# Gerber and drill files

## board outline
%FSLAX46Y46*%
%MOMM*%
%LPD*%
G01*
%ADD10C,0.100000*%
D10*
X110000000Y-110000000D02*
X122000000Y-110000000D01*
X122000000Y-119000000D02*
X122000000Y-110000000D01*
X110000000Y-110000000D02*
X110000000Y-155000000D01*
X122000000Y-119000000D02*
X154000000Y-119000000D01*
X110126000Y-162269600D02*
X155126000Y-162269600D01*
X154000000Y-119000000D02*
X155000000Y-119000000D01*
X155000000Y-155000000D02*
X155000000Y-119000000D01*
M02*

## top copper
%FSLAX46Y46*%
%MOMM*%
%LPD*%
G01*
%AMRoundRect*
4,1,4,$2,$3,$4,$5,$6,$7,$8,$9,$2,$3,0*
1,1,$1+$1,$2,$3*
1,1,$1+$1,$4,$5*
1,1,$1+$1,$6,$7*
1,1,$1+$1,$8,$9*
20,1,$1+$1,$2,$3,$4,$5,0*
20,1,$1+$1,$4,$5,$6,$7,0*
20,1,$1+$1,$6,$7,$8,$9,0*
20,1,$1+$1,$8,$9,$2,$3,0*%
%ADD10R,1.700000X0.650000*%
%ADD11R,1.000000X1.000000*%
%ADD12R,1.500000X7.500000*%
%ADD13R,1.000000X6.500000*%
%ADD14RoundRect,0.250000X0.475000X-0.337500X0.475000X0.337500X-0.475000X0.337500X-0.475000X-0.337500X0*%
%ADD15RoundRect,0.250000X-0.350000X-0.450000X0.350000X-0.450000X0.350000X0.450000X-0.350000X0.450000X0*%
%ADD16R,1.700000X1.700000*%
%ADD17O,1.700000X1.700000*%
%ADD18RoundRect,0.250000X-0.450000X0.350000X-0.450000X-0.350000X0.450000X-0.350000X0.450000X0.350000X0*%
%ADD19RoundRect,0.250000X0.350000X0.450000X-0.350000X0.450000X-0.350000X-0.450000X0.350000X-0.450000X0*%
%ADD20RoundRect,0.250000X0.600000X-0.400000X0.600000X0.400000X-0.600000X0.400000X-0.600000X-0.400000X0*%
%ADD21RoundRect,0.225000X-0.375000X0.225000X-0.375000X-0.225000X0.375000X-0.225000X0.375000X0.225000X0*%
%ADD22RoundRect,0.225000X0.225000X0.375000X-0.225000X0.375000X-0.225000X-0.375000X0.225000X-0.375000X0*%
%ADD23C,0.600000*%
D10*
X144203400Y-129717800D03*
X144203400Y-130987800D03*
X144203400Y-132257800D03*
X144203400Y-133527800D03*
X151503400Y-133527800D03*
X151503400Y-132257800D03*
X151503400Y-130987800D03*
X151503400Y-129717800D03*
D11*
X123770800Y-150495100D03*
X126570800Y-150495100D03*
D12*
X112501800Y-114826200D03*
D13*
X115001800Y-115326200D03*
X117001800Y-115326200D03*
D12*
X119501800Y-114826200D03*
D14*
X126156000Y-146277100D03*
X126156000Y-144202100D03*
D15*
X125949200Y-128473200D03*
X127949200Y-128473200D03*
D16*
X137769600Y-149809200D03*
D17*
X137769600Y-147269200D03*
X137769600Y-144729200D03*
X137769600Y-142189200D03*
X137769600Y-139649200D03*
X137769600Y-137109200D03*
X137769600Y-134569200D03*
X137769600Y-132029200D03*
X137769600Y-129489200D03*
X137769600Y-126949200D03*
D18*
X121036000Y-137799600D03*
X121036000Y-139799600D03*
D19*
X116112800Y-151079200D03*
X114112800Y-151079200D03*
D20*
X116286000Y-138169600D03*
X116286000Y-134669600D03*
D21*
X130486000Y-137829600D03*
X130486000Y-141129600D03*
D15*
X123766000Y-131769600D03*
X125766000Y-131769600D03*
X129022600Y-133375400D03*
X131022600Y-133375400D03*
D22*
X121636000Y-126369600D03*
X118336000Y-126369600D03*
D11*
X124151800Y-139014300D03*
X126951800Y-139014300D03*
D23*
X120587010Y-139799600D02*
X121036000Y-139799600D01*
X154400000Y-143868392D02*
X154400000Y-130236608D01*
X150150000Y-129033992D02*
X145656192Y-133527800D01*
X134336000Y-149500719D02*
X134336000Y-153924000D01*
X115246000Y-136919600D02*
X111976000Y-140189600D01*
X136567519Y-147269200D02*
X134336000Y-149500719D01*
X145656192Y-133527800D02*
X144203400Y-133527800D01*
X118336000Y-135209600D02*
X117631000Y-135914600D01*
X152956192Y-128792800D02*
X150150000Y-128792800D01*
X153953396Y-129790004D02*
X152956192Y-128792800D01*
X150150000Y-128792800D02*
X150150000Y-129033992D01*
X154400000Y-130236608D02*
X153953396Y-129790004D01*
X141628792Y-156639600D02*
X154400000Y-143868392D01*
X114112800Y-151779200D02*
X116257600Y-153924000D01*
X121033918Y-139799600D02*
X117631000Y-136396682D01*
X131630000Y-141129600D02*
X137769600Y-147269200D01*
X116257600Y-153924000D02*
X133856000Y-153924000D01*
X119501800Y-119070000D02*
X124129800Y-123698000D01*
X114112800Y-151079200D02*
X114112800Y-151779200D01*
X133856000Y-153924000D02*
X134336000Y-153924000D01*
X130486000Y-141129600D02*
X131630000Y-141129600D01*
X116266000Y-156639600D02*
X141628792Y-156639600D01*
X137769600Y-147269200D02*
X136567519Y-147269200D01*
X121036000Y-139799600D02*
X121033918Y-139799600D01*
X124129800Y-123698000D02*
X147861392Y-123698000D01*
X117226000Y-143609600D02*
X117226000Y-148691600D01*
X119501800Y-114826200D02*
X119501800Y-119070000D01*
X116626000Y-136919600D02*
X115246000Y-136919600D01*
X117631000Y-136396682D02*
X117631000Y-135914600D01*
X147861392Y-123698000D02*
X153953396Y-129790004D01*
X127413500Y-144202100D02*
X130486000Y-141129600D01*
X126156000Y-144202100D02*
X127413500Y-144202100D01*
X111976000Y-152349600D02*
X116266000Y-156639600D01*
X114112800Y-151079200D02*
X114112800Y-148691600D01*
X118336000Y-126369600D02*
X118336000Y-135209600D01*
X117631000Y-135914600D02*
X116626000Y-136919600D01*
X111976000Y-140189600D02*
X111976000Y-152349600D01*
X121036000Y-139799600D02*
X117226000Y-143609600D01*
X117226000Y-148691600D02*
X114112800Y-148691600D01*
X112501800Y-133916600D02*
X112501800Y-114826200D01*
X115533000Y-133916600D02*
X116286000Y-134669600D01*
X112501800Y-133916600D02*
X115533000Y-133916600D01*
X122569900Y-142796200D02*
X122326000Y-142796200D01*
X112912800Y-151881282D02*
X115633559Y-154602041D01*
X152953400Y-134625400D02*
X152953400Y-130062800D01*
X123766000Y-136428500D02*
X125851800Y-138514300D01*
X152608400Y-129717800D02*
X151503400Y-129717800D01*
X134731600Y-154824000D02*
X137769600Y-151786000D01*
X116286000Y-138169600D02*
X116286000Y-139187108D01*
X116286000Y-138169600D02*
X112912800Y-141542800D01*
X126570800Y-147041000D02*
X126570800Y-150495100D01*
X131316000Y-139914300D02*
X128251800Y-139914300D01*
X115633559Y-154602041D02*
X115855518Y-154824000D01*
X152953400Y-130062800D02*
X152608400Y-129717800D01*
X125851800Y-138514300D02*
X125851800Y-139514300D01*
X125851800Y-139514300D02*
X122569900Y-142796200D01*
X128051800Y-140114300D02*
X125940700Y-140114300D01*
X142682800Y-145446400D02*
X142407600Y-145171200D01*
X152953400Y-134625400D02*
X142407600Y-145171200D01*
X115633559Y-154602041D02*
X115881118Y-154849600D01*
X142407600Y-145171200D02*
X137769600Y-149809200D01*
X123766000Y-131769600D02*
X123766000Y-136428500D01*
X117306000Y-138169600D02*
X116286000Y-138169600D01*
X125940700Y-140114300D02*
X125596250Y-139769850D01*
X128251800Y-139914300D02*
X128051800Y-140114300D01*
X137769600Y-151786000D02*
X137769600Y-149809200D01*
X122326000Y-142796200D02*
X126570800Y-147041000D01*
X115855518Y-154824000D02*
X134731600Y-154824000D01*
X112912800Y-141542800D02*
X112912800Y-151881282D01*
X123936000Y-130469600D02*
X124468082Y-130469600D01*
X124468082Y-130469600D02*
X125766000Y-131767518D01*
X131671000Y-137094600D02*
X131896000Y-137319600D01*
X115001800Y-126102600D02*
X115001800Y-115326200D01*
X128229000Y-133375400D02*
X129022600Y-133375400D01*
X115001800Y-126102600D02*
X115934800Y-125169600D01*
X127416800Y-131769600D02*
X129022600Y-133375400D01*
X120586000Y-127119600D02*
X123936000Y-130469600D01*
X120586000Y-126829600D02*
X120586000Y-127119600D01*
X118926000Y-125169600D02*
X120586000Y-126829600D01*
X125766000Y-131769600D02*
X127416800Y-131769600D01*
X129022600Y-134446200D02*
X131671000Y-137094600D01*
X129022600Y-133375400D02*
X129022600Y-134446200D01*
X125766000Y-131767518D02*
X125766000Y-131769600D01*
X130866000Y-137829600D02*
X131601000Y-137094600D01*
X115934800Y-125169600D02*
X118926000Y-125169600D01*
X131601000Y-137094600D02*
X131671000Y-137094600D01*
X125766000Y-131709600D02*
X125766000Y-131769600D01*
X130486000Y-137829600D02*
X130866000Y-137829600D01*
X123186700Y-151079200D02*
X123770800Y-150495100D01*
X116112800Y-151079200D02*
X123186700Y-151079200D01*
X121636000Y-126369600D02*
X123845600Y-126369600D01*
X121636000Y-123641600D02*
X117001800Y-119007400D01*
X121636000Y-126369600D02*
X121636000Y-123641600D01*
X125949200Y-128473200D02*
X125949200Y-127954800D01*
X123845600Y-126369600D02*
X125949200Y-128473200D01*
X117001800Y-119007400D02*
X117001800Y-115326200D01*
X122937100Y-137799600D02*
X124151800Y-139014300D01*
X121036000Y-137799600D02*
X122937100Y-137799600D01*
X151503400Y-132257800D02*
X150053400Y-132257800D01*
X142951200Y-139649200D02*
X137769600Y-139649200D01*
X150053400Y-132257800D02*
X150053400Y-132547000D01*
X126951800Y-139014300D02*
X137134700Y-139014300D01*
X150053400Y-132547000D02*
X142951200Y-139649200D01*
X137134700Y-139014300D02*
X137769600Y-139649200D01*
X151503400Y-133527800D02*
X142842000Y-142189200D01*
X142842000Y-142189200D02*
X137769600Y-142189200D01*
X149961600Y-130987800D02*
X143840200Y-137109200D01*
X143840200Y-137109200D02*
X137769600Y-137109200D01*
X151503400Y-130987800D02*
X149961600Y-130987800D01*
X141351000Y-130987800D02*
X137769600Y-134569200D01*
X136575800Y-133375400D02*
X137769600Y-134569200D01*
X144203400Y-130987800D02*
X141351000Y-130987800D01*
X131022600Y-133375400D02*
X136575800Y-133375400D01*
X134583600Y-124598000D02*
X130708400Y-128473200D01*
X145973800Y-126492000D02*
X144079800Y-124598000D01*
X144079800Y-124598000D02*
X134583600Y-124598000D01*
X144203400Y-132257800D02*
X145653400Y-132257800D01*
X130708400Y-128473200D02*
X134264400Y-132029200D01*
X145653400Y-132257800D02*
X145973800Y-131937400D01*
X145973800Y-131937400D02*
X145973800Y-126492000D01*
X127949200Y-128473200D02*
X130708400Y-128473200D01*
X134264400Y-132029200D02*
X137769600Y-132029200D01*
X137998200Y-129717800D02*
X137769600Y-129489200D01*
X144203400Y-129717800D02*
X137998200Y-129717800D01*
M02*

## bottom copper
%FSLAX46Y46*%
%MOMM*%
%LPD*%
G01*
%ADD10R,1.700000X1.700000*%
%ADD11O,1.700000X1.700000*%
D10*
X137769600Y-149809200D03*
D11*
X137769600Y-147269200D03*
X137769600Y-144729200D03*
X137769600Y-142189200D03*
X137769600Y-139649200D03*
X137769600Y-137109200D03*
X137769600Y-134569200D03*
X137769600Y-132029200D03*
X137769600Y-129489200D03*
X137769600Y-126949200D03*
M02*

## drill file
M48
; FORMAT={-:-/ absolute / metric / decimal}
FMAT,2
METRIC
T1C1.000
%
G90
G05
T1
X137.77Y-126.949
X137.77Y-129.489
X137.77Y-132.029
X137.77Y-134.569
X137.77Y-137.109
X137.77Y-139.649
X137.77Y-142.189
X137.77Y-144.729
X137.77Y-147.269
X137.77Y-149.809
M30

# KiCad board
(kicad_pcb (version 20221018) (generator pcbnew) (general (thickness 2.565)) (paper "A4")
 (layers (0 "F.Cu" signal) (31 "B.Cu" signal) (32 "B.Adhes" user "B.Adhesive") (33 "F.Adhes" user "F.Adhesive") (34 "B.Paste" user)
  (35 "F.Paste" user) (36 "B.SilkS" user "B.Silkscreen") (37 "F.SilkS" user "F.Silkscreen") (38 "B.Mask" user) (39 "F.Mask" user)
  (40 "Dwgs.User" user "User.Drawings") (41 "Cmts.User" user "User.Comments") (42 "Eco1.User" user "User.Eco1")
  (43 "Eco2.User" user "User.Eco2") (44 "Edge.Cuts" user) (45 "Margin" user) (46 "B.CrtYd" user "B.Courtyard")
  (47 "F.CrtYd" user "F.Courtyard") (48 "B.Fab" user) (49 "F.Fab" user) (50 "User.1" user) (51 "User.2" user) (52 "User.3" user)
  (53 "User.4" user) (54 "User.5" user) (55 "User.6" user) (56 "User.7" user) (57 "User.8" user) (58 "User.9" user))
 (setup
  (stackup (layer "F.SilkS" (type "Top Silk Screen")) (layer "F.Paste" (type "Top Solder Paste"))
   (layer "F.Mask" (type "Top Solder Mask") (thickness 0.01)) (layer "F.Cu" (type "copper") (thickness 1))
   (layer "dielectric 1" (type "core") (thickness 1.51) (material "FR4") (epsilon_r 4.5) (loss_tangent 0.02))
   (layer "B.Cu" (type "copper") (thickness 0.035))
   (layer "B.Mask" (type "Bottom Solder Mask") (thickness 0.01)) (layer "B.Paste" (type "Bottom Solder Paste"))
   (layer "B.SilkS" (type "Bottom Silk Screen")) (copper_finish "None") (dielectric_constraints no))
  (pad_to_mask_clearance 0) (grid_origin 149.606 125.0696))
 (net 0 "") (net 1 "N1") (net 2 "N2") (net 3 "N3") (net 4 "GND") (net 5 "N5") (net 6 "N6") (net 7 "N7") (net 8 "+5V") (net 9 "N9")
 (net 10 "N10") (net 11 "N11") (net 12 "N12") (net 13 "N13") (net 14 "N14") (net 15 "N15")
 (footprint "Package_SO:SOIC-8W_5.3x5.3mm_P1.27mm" (layer "F.Cu") (at 147.8534 131.6228)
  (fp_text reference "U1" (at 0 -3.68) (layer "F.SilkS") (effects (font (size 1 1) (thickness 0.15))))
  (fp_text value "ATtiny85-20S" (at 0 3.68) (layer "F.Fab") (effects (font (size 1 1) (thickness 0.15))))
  (pad "1" smd rect (at -3.65 -1.905) (size 1.7 0.65) (layers "F.Cu" "F.Paste" "F.Mask") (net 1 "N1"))
  (pad "2" smd rect (at -3.65 -0.635) (size 1.7 0.65) (layers "F.Cu" "F.Paste" "F.Mask") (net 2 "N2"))
  (pad "3" smd rect (at -3.65 0.635) (size 1.7 0.65) (layers "F.Cu" "F.Paste" "F.Mask") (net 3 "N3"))
  (pad "4" smd rect (at -3.65 1.905) (size 1.7 0.65) (layers "F.Cu" "F.Paste" "F.Mask") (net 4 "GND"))
  (pad "5" smd rect (at 3.65 1.905) (size 1.7 0.65) (layers "F.Cu" "F.Paste" "F.Mask") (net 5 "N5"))
  (pad "6" smd rect (at 3.65 0.635) (size 1.7 0.65) (layers "F.Cu" "F.Paste" "F.Mask") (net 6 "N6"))
  (pad "7" smd rect (at 3.65 -0.635) (size 1.7 0.65) (layers "F.Cu" "F.Paste" "F.Mask") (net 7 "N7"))
  (pad "8" smd rect (at 3.65 -1.905) (size 1.7 0.65) (layers "F.Cu" "F.Paste" "F.Mask") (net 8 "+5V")))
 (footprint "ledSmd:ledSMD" (layer "F.Cu") (at 125.5708 150.4951)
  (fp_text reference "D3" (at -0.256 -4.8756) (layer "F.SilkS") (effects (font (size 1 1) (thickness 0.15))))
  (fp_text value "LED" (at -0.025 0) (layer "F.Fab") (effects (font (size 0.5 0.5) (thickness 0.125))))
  (pad "1" smd rect (at -1.8 0) (size 1 1) (layers "F.Cu" "F.Paste" "F.Mask") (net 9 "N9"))
  (pad "2" smd rect (at 1 0) (size 1 1) (layers "F.Cu" "F.Paste" "F.Mask") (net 8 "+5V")))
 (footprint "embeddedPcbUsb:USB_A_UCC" (layer "F.Cu") (at 116.0018 115.0262 -90)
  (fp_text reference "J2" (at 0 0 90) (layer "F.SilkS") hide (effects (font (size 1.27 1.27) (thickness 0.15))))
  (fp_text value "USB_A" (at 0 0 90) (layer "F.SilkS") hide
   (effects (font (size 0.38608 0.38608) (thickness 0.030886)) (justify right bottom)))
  (pad "1" smd rect (at -0.2 3.5 270) (size 7.5 1.5) (layers "F.Cu" "F.Paste" "F.Mask") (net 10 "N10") (solder_mask_margin 0.1016))
  (pad "2" smd rect (at 0.3 1 270) (size 6.5 1) (layers "F.Cu" "F.Paste" "F.Mask") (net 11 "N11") (solder_mask_margin 0.1016))
  (pad "3" smd rect (at 0.3 -1 270) (size 6.5 1) (layers "F.Cu" "F.Paste" "F.Mask") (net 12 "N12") (solder_mask_margin 0.1016))
  (pad "4" smd rect (at -0.2 -3.5 270) (size 7.5 1.5) (layers "F.Cu" "F.Paste" "F.Mask") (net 4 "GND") (solder_mask_margin 0.1016)))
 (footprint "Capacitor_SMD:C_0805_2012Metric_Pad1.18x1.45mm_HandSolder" (layer "F.Cu") (at 126.156 145.2396 90)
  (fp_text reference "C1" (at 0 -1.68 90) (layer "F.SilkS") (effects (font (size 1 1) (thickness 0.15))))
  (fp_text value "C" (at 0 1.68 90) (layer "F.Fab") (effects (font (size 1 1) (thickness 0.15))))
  (pad "1" smd roundrect (at -1.0375 0 90) (size 1.175 1.45) (layers "F.Cu" "F.Paste" "F.Mask") (roundrect_rratio 0.212766) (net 8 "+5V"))
  (pad "2" smd roundrect (at 1.0375 0 90) (size 1.175 1.45) (layers "F.Cu" "F.Paste" "F.Mask") (roundrect_rratio 0.212766) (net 4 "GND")))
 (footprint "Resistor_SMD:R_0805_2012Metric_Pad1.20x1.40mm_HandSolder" (layer "F.Cu") (at 126.9492 128.4732)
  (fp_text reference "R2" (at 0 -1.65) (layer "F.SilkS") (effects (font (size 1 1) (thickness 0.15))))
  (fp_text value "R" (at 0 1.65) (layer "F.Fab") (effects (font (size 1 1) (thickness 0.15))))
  (pad "1" smd roundrect (at -1 0) (size 1.2 1.4) (layers "F.Cu" "F.Paste" "F.Mask") (roundrect_rratio 0.208333) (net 12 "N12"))
  (pad "2" smd roundrect (at 1 0) (size 1.2 1.4) (layers "F.Cu" "F.Paste" "F.Mask") (roundrect_rratio 0.208333) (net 3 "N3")))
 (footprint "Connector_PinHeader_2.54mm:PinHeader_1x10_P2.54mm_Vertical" (layer "F.Cu") (at 137.7696 149.8092 180)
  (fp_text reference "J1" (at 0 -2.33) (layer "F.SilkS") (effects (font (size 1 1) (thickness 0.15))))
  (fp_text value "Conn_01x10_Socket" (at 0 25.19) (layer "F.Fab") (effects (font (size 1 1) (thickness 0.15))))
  (pad "1" thru_hole rect (at 0 0 180) (size 1.7 1.7) (drill 1) (layers "*.Cu" "*.Mask") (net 8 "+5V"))
  (pad "2" thru_hole oval (at 0 2.54 180) (size 1.7 1.7) (drill 1) (layers "*.Cu" "*.Mask") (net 4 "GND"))
  (pad "3" thru_hole oval (at 0 5.08 180) (size 1.7 1.7) (drill 1) (layers "*.Cu" "*.Mask") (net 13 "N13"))
  (pad "4" thru_hole oval (at 0 7.62 180) (size 1.7 1.7) (drill 1) (layers "*.Cu" "*.Mask") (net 5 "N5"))
  (pad "5" thru_hole oval (at 0 10.16 180) (size 1.7 1.7) (drill 1) (layers "*.Cu" "*.Mask") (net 6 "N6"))
  (pad "6" thru_hole oval (at 0 12.7 180) (size 1.7 1.7) (drill 1) (layers "*.Cu" "*.Mask") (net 7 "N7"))
  (pad "7" thru_hole oval (at 0 15.24 180) (size 1.7 1.7) (drill 1) (layers "*.Cu" "*.Mask") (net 2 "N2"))
  (pad "8" thru_hole oval (at 0 17.78 180) (size 1.7 1.7) (drill 1) (layers "*.Cu" "*.Mask") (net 3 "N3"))
  (pad "9" thru_hole oval (at 0 20.32 180) (size 1.7 1.7) (drill 1) (layers "*.Cu" "*.Mask") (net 1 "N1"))
  (pad "10" thru_hole oval (at 0 22.86 180) (size 1.7 1.7) (drill 1) (layers "*.Cu" "*.Mask") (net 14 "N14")))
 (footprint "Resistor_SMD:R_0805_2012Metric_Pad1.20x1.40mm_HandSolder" (layer "F.Cu") (at 121.036 138.7996 -90)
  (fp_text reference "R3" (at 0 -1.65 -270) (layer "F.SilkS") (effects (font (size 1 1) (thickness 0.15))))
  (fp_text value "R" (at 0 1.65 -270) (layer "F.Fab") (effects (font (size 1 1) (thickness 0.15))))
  (pad "1" smd roundrect (at -1 0 270) (size 1.2 1.4) (layers "F.Cu" "F.Paste" "F.Mask") (roundrect_rratio 0.208333) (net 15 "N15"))
  (pad "2" smd roundrect (at 1 0 270) (size 1.2 1.4) (layers "F.Cu" "F.Paste" "F.Mask") (roundrect_rratio 0.208333) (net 4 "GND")))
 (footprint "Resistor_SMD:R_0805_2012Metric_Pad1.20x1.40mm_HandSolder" (layer "F.Cu") (at 115.1128 151.0792 180)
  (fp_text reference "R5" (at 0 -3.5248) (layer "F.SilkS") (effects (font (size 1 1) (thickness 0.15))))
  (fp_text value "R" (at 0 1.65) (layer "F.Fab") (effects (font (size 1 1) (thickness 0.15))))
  (pad "1" smd roundrect (at -1 0 180) (size 1.2 1.4) (layers "F.Cu" "F.Paste" "F.Mask") (roundrect_rratio 0.208333) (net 9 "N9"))
  (pad "2" smd roundrect (at 1 0 180) (size 1.2 1.4) (layers "F.Cu" "F.Paste" "F.Mask") (roundrect_rratio 0.208333) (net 4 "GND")))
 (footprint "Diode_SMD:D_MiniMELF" (layer "F.Cu") (at 116.286 136.4196 90)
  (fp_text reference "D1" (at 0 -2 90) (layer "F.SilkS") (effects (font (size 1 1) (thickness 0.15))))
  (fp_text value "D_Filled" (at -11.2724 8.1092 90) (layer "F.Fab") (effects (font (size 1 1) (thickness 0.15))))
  (pad "1" smd roundrect (at -1.75 0 90) (size 1.3 1.7) (layers "F.Cu" "F.Paste" "F.Mask") (roundrect_rratio 0.1923076923) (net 8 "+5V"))
  (pad "2" smd roundrect (at 1.75 0 90) (size 1.3 1.7) (layers "F.Cu" "F.Paste" "F.Mask") (roundrect_rratio 0.1923076923) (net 10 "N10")))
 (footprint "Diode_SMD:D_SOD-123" (layer "F.Cu") (at 130.486 139.4796 -90)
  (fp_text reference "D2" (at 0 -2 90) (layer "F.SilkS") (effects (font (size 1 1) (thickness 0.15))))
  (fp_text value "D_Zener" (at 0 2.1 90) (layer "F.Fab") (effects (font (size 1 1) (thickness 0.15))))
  (pad "1" smd roundrect (at -1.65 0 270) (size 0.9 1.2) (layers "F.Cu" "F.Paste" "F.Mask") (roundrect_rratio 0.25) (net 11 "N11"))
  (pad "2" smd roundrect (at 1.65 0 270) (size 0.9 1.2) (layers "F.Cu" "F.Paste" "F.Mask") (roundrect_rratio 0.25) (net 4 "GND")))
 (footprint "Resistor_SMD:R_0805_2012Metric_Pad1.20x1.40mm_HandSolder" (layer "F.Cu") (at 124.766 131.7696)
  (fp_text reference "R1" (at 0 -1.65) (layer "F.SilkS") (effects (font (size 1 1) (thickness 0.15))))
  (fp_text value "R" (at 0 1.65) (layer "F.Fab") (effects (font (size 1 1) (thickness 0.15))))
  (pad "1" smd roundrect (at -1 0) (size 1.2 1.4) (layers "F.Cu" "F.Paste" "F.Mask") (roundrect_rratio 0.208333) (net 8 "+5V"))
  (pad "2" smd roundrect (at 1 0) (size 1.2 1.4) (layers "F.Cu" "F.Paste" "F.Mask") (roundrect_rratio 0.208333) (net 11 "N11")))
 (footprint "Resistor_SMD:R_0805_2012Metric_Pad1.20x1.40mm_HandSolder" (layer "F.Cu") (at 130.0226 133.3754)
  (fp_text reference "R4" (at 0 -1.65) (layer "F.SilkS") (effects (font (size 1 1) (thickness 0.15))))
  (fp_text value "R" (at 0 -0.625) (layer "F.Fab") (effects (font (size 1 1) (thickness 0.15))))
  (pad "1" smd roundrect (at -1 0) (size 1.2 1.4) (layers "F.Cu" "F.Paste" "F.Mask") (roundrect_rratio 0.208333) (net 11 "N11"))
  (pad "2" smd roundrect (at 1 0) (size 1.2 1.4) (layers "F.Cu" "F.Paste" "F.Mask") (roundrect_rratio 0.208333) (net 2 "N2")))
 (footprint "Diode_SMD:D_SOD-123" (layer "F.Cu") (at 119.986 126.3696 180)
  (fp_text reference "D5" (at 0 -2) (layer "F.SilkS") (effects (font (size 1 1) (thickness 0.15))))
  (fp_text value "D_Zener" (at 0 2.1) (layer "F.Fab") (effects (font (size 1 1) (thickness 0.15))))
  (pad "1" smd roundrect (at -1.65 0 180) (size 0.9 1.2) (layers "F.Cu" "F.Paste" "F.Mask") (roundrect_rratio 0.25) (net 12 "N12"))
  (pad "2" smd roundrect (at 1.65 0 180) (size 0.9 1.2) (layers "F.Cu" "F.Paste" "F.Mask") (roundrect_rratio 0.25) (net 4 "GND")))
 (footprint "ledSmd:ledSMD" (layer "F.Cu") (at 125.9518 139.0143)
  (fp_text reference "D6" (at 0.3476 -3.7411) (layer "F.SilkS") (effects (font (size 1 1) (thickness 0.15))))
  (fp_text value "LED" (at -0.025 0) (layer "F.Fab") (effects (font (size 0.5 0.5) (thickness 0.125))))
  (pad "1" smd rect (at -1.8 0) (size 1 1) (layers "F.Cu" "F.Paste" "F.Mask") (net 15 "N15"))
  (pad "2" smd rect (at 1 0) (size 1 1) (layers "F.Cu" "F.Paste" "F.Mask") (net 6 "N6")))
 (gr_line (start 110 110) (end 122 110) (stroke (width 0.1) (type default)) (layer "Edge.Cuts"))
 (gr_line (start 122 119) (end 122 110) (stroke (width 0.1) (type default)) (layer "Edge.Cuts"))
 (gr_line (start 110 110) (end 110 155) (stroke (width 0.1) (type default)) (layer "Edge.Cuts"))
 (gr_line (start 122 119) (end 154 119) (stroke (width 0.1) (type default)) (layer "Edge.Cuts"))
 (gr_line (start 110.126 162.2696) (end 155.126 162.2696) (stroke (width 0.1) (type default)) (layer "Edge.Cuts"))
 (gr_line (start 154 119) (end 155 119) (stroke (width 0.1) (type default)) (layer "Edge.Cuts"))
 (gr_line (start 155 155) (end 155 119) (stroke (width 0.1) (type default)) (layer "Edge.Cuts"))
 (segment (start 120.58701 139.7996) (end 121.036 139.7996) (width 0.6) (layer "F.Cu") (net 4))
 (segment (start 154.4 143.868392) (end 154.4 130.236608) (width 0.6) (layer "F.Cu") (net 4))
 (segment (start 150.15 129.033992) (end 145.656192 133.5278) (width 0.6) (layer "F.Cu") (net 4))
 (segment (start 134.336 149.500719) (end 134.336 153.924) (width 0.6) (layer "F.Cu") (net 4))
 (segment (start 115.246 136.9196) (end 111.976 140.1896) (width 0.6) (layer "F.Cu") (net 4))
 (segment (start 136.567519 147.2692) (end 134.336 149.500719) (width 0.6) (layer "F.Cu") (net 4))
 (segment (start 145.656192 133.5278) (end 144.2034 133.5278) (width 0.6) (layer "F.Cu") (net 4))
 (segment (start 118.336 135.2096) (end 117.631 135.9146) (width 0.6) (layer "F.Cu") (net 4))
 (segment (start 152.956192 128.7928) (end 150.15 128.7928) (width 0.6) (layer "F.Cu") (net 4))
 (segment (start 153.953396 129.790004) (end 152.956192 128.7928) (width 0.6) (layer "F.Cu") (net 4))
 (segment (start 150.15 128.7928) (end 150.15 129.033992) (width 0.6) (layer "F.Cu") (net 4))
 (segment (start 154.4 130.236608) (end 153.953396 129.790004) (width 0.6) (layer "F.Cu") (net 4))
 (segment (start 141.628792 156.6396) (end 154.4 143.868392) (width 0.6) (layer "F.Cu") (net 4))
 (segment (start 114.1128 151.7792) (end 116.2576 153.924) (width 0.6) (layer "F.Cu") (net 4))
 (segment (start 121.033918 139.7996) (end 117.631 136.396682) (width 0.6) (layer "F.Cu") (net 4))
 (segment (start 131.63 141.1296) (end 137.7696 147.2692) (width 0.6) (layer "F.Cu") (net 4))
 (segment (start 116.2576 153.924) (end 133.856 153.924) (width 0.6) (layer "F.Cu") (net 4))
 (segment (start 119.5018 119.07) (end 124.1298 123.698) (width 0.6) (layer "F.Cu") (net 4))
 (segment (start 114.1128 151.0792) (end 114.1128 151.7792) (width 0.6) (layer "F.Cu") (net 4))
 (segment (start 133.856 153.924) (end 134.336 153.924) (width 0.6) (layer "F.Cu") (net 4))
 (segment (start 130.486 141.1296) (end 131.63 141.1296) (width 0.6) (layer "F.Cu") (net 4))
 (segment (start 116.266 156.6396) (end 141.628792 156.6396) (width 0.6) (layer "F.Cu") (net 4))
 (segment (start 137.7696 147.2692) (end 136.567519 147.2692) (width 0.6) (layer "F.Cu") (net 4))
 (segment (start 121.036 139.7996) (end 121.033918 139.7996) (width 0.6) (layer "F.Cu") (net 4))
 (segment (start 124.1298 123.698) (end 147.861392 123.698) (width 0.6) (layer "F.Cu") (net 4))
 (segment (start 117.226 143.6096) (end 117.226 148.6916) (width 0.6) (layer "F.Cu") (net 4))
 (segment (start 119.5018 114.8262) (end 119.5018 119.07) (width 0.6) (layer "F.Cu") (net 4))
 (segment (start 116.626 136.9196) (end 115.246 136.9196) (width 0.6) (layer "F.Cu") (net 4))
 (segment (start 117.631 136.396682) (end 117.631 135.9146) (width 0.6) (layer "F.Cu") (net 4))
 (segment (start 147.861392 123.698) (end 153.953396 129.790004) (width 0.6) (layer "F.Cu") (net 4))
 (segment (start 127.4135 144.2021) (end 130.486 141.1296) (width 0.6) (layer "F.Cu") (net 4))
 (segment (start 126.156 144.2021) (end 127.4135 144.2021) (width 0.6) (layer "F.Cu") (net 4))
 (segment (start 111.976 152.3496) (end 116.266 156.6396) (width 0.6) (layer "F.Cu") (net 4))
 (segment (start 114.1128 151.0792) (end 114.1128 148.6916) (width 0.6) (layer "F.Cu") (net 4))
 (segment (start 118.336 126.3696) (end 118.336 135.2096) (width 0.6) (layer "F.Cu") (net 4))
 (segment (start 117.631 135.9146) (end 116.626 136.9196) (width 0.6) (layer "F.Cu") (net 4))
 (segment (start 111.976 140.1896) (end 111.976 152.3496) (width 0.6) (layer "F.Cu") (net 4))
 (segment (start 121.036 139.7996) (end 117.226 143.6096) (width 0.6) (layer "F.Cu") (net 4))
 (segment (start 117.226 148.6916) (end 114.1128 148.6916) (width 0.6) (layer "F.Cu") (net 4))
 (segment (start 112.5018 133.9166) (end 112.5018 114.8262) (width 0.6) (layer "F.Cu") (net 10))
 (segment (start 115.533 133.9166) (end 116.286 134.6696) (width 0.6) (layer "F.Cu") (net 10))
 (segment (start 112.5018 133.9166) (end 115.533 133.9166) (width 0.6) (layer "F.Cu") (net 10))
 (segment (start 122.5699 142.7962) (end 122.326 142.7962) (width 0.6) (layer "F.Cu") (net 8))
 (segment (start 112.9128 151.881282) (end 115.633559 154.602041) (width 0.6) (layer "F.Cu") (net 8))
 (segment (start 152.9534 134.6254) (end 152.9534 130.0628) (width 0.6) (layer "F.Cu") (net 8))
 (segment (start 123.766 136.4285) (end 125.8518 138.5143) (width 0.6) (layer "F.Cu") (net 8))
 (segment (start 152.6084 129.7178) (end 151.5034 129.7178) (width 0.6) (layer "F.Cu") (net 8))
 (segment (start 134.7316 154.824) (end 137.7696 151.786) (width 0.6) (layer "F.Cu") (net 8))
 (segment (start 116.286 138.1696) (end 116.286 139.187108) (width 0.6) (layer "F.Cu") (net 8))
 (segment (start 116.286 138.1696) (end 112.9128 141.5428) (width 0.6) (layer "F.Cu") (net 8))
 (segment (start 126.5708 147.041) (end 126.5708 150.4951) (width 0.6) (layer "F.Cu") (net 8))
 (segment (start 131.316 139.9143) (end 128.2518 139.9143) (width 0.6) (layer "F.Cu") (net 8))
 (segment (start 115.633559 154.602041) (end 115.855518 154.824) (width 0.6) (layer "F.Cu") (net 8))
 (segment (start 152.9534 130.0628) (end 152.6084 129.7178) (width 0.6) (layer "F.Cu") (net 8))
 (segment (start 125.8518 138.5143) (end 125.8518 139.5143) (width 0.6) (layer "F.Cu") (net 8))
 (segment (start 125.8518 139.5143) (end 122.5699 142.7962) (width 0.6) (layer "F.Cu") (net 8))
 (segment (start 128.0518 140.1143) (end 125.9407 140.1143) (width 0.6) (layer "F.Cu") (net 8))
 (segment (start 142.6828 145.4464) (end 142.4076 145.1712) (width 0.6) (layer "F.Cu") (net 8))
 (segment (start 152.9534 134.6254) (end 142.4076 145.1712) (width 0.6) (layer "F.Cu") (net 8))
 (segment (start 115.633559 154.602041) (end 115.881118 154.8496) (width 0.6) (layer "F.Cu") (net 8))
 (segment (start 142.4076 145.1712) (end 137.7696 149.8092) (width 0.6) (layer "F.Cu") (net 8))
 (segment (start 123.766 131.7696) (end 123.766 136.4285) (width 0.6) (layer "F.Cu") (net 8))
 (segment (start 117.306 138.1696) (end 116.286 138.1696) (width 0.6) (layer "F.Cu") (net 8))
 (segment (start 125.9407 140.1143) (end 125.59625 139.76985) (width 0.6) (layer "F.Cu") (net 8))
 (segment (start 128.2518 139.9143) (end 128.0518 140.1143) (width 0.6) (layer "F.Cu") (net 8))
 (segment (start 137.7696 151.786) (end 137.7696 149.8092) (width 0.6) (layer "F.Cu") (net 8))
 (segment (start 122.326 142.7962) (end 126.5708 147.041) (width 0.6) (layer "F.Cu") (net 8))
 (segment (start 115.855518 154.824) (end 134.7316 154.824) (width 0.6) (layer "F.Cu") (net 8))
 (segment (start 112.9128 141.5428) (end 112.9128 151.881282) (width 0.6) (layer "F.Cu") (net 8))
 (segment (start 123.936 130.4696) (end 124.468082 130.4696) (width 0.6) (layer "F.Cu") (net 11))
 (segment (start 124.468082 130.4696) (end 125.766 131.767518) (width 0.6) (layer "F.Cu") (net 11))
 (segment (start 131.671 137.0946) (end 131.896 137.3196) (width 0.6) (layer "F.Cu") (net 11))
 (segment (start 115.0018 126.1026) (end 115.0018 115.3262) (width 0.6) (layer "F.Cu") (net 11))
 (segment (start 128.229 133.3754) (end 129.0226 133.3754) (width 0.6) (layer "F.Cu") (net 11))
 (segment (start 115.0018 126.1026) (end 115.9348 125.1696) (width 0.6) (layer "F.Cu") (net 11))
 (segment (start 127.4168 131.7696) (end 129.0226 133.3754) (width 0.6) (layer "F.Cu") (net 11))
 (segment (start 120.586 127.1196) (end 123.936 130.4696) (width 0.6) (layer "F.Cu") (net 11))
 (segment (start 120.586 126.8296) (end 120.586 127.1196) (width 0.6) (layer "F.Cu") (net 11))
 (segment (start 118.926 125.1696) (end 120.586 126.8296) (width 0.6) (layer "F.Cu") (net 11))
 (segment (start 125.766 131.7696) (end 127.4168 131.7696) (width 0.6) (layer "F.Cu") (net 11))
 (segment (start 129.0226 134.4462) (end 131.671 137.0946) (width 0.6) (layer "F.Cu") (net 11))
 (segment (start 129.0226 133.3754) (end 129.0226 134.4462) (width 0.6) (layer "F.Cu") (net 11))
 (segment (start 125.766 131.767518) (end 125.766 131.7696) (width 0.6) (layer "F.Cu") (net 11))
 (segment (start 130.866 137.8296) (end 131.601 137.0946) (width 0.6) (layer "F.Cu") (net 11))
 (segment (start 115.9348 125.1696) (end 118.926 125.1696) (width 0.6) (layer "F.Cu") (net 11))
 (segment (start 131.601 137.0946) (end 131.671 137.0946) (width 0.6) (layer "F.Cu") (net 11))
 (segment (start 125.766 131.7096) (end 125.766 131.7696) (width 0.6) (layer "F.Cu") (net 11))
 (segment (start 130.486 137.8296) (end 130.866 137.8296) (width 0.6) (layer "F.Cu") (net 11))
 (segment (start 123.1867 151.0792) (end 123.7708 150.4951) (width 0.6) (layer "F.Cu") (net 9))
 (segment (start 116.1128 151.0792) (end 123.1867 151.0792) (width 0.6) (layer "F.Cu") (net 9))
 (segment (start 121.636 126.3696) (end 123.8456 126.3696) (width 0.6) (layer "F.Cu") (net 12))
 (segment (start 121.636 123.6416) (end 117.0018 119.0074) (width 0.6) (layer "F.Cu") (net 12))
 (segment (start 121.636 126.3696) (end 121.636 123.6416) (width 0.6) (layer "F.Cu") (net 12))
 (segment (start 125.9492 128.4732) (end 125.9492 127.9548) (width 0.6) (layer "F.Cu") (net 12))
 (segment (start 123.8456 126.3696) (end 125.9492 128.4732) (width 0.6) (layer "F.Cu") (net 12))
 (segment (start 117.0018 119.0074) (end 117.0018 115.3262) (width 0.6) (layer "F.Cu") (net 12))
 (segment (start 122.9371 137.7996) (end 124.1518 139.0143) (width 0.6) (layer "F.Cu") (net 15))
 (segment (start 121.036 137.7996) (end 122.9371 137.7996) (width 0.6) (layer "F.Cu") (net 15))
 (segment (start 151.5034 132.2578) (end 150.0534 132.2578) (width 0.6) (layer "F.Cu") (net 6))
 (segment (start 142.9512 139.6492) (end 137.7696 139.6492) (width 0.6) (layer "F.Cu") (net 6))
 (segment (start 150.0534 132.2578) (end 150.0534 132.547) (width 0.6) (layer "F.Cu") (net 6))
 (segment (start 126.9518 139.0143) (end 137.1347 139.0143) (width 0.6) (layer "F.Cu") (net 6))
 (segment (start 150.0534 132.547) (end 142.9512 139.6492) (width 0.6) (layer "F.Cu") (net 6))
 (segment (start 137.1347 139.0143) (end 137.7696 139.6492) (width 0.6) (layer "F.Cu") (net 6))
 (segment (start 151.5034 133.5278) (end 142.842 142.1892) (width 0.6) (layer "F.Cu") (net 5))
 (segment (start 142.842 142.1892) (end 137.7696 142.1892) (width 0.6) (layer "F.Cu") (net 5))
 (segment (start 149.9616 130.9878) (end 143.8402 137.1092) (width 0.6) (layer "F.Cu") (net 7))
 (segment (start 143.8402 137.1092) (end 137.7696 137.1092) (width 0.6) (layer "F.Cu") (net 7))
 (segment (start 151.5034 130.9878) (end 149.9616 130.9878) (width 0.6) (layer "F.Cu") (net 7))
 (segment (start 141.351 130.9878) (end 137.7696 134.5692) (width 0.6) (layer "F.Cu") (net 2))
 (segment (start 136.5758 133.3754) (end 137.7696 134.5692) (width 0.6) (layer "F.Cu") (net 2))
 (segment (start 144.2034 130.9878) (end 141.351 130.9878) (width 0.6) (layer "F.Cu") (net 2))
 (segment (start 131.0226 133.3754) (end 136.5758 133.3754) (width 0.6) (layer "F.Cu") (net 2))
 (segment (start 134.5836 124.598) (end 130.7084 128.4732) (width 0.6) (layer "F.Cu") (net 3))
 (segment (start 145.9738 126.492) (end 144.0798 124.598) (width 0.6) (layer "F.Cu") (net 3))
 (segment (start 144.0798 124.598) (end 134.5836 124.598) (width 0.6) (layer "F.Cu") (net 3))
 (segment (start 144.2034 132.2578) (end 145.6534 132.2578) (width 0.6) (layer "F.Cu") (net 3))
 (segment (start 130.7084 128.4732) (end 134.2644 132.0292) (width 0.6) (layer "F.Cu") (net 3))
 (segment (start 145.6534 132.2578) (end 145.9738 131.9374) (width 0.6) (layer "F.Cu") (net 3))
 (segment (start 145.9738 131.9374) (end 145.9738 126.492) (width 0.6) (layer "F.Cu") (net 3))
 (segment (start 127.9492 128.4732) (end 130.7084 128.4732) (width 0.6) (layer "F.Cu") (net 3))
 (segment (start 134.2644 132.0292) (end 137.7696 132.0292) (width 0.6) (layer "F.Cu") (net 3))
 (segment (start 137.9982 129.7178) (end 137.7696 129.4892) (width 0.6) (layer "F.Cu") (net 1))
 (segment (start 144.2034 129.7178) (end 137.9982 129.7178) (width 0.6) (layer "F.Cu") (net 1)))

